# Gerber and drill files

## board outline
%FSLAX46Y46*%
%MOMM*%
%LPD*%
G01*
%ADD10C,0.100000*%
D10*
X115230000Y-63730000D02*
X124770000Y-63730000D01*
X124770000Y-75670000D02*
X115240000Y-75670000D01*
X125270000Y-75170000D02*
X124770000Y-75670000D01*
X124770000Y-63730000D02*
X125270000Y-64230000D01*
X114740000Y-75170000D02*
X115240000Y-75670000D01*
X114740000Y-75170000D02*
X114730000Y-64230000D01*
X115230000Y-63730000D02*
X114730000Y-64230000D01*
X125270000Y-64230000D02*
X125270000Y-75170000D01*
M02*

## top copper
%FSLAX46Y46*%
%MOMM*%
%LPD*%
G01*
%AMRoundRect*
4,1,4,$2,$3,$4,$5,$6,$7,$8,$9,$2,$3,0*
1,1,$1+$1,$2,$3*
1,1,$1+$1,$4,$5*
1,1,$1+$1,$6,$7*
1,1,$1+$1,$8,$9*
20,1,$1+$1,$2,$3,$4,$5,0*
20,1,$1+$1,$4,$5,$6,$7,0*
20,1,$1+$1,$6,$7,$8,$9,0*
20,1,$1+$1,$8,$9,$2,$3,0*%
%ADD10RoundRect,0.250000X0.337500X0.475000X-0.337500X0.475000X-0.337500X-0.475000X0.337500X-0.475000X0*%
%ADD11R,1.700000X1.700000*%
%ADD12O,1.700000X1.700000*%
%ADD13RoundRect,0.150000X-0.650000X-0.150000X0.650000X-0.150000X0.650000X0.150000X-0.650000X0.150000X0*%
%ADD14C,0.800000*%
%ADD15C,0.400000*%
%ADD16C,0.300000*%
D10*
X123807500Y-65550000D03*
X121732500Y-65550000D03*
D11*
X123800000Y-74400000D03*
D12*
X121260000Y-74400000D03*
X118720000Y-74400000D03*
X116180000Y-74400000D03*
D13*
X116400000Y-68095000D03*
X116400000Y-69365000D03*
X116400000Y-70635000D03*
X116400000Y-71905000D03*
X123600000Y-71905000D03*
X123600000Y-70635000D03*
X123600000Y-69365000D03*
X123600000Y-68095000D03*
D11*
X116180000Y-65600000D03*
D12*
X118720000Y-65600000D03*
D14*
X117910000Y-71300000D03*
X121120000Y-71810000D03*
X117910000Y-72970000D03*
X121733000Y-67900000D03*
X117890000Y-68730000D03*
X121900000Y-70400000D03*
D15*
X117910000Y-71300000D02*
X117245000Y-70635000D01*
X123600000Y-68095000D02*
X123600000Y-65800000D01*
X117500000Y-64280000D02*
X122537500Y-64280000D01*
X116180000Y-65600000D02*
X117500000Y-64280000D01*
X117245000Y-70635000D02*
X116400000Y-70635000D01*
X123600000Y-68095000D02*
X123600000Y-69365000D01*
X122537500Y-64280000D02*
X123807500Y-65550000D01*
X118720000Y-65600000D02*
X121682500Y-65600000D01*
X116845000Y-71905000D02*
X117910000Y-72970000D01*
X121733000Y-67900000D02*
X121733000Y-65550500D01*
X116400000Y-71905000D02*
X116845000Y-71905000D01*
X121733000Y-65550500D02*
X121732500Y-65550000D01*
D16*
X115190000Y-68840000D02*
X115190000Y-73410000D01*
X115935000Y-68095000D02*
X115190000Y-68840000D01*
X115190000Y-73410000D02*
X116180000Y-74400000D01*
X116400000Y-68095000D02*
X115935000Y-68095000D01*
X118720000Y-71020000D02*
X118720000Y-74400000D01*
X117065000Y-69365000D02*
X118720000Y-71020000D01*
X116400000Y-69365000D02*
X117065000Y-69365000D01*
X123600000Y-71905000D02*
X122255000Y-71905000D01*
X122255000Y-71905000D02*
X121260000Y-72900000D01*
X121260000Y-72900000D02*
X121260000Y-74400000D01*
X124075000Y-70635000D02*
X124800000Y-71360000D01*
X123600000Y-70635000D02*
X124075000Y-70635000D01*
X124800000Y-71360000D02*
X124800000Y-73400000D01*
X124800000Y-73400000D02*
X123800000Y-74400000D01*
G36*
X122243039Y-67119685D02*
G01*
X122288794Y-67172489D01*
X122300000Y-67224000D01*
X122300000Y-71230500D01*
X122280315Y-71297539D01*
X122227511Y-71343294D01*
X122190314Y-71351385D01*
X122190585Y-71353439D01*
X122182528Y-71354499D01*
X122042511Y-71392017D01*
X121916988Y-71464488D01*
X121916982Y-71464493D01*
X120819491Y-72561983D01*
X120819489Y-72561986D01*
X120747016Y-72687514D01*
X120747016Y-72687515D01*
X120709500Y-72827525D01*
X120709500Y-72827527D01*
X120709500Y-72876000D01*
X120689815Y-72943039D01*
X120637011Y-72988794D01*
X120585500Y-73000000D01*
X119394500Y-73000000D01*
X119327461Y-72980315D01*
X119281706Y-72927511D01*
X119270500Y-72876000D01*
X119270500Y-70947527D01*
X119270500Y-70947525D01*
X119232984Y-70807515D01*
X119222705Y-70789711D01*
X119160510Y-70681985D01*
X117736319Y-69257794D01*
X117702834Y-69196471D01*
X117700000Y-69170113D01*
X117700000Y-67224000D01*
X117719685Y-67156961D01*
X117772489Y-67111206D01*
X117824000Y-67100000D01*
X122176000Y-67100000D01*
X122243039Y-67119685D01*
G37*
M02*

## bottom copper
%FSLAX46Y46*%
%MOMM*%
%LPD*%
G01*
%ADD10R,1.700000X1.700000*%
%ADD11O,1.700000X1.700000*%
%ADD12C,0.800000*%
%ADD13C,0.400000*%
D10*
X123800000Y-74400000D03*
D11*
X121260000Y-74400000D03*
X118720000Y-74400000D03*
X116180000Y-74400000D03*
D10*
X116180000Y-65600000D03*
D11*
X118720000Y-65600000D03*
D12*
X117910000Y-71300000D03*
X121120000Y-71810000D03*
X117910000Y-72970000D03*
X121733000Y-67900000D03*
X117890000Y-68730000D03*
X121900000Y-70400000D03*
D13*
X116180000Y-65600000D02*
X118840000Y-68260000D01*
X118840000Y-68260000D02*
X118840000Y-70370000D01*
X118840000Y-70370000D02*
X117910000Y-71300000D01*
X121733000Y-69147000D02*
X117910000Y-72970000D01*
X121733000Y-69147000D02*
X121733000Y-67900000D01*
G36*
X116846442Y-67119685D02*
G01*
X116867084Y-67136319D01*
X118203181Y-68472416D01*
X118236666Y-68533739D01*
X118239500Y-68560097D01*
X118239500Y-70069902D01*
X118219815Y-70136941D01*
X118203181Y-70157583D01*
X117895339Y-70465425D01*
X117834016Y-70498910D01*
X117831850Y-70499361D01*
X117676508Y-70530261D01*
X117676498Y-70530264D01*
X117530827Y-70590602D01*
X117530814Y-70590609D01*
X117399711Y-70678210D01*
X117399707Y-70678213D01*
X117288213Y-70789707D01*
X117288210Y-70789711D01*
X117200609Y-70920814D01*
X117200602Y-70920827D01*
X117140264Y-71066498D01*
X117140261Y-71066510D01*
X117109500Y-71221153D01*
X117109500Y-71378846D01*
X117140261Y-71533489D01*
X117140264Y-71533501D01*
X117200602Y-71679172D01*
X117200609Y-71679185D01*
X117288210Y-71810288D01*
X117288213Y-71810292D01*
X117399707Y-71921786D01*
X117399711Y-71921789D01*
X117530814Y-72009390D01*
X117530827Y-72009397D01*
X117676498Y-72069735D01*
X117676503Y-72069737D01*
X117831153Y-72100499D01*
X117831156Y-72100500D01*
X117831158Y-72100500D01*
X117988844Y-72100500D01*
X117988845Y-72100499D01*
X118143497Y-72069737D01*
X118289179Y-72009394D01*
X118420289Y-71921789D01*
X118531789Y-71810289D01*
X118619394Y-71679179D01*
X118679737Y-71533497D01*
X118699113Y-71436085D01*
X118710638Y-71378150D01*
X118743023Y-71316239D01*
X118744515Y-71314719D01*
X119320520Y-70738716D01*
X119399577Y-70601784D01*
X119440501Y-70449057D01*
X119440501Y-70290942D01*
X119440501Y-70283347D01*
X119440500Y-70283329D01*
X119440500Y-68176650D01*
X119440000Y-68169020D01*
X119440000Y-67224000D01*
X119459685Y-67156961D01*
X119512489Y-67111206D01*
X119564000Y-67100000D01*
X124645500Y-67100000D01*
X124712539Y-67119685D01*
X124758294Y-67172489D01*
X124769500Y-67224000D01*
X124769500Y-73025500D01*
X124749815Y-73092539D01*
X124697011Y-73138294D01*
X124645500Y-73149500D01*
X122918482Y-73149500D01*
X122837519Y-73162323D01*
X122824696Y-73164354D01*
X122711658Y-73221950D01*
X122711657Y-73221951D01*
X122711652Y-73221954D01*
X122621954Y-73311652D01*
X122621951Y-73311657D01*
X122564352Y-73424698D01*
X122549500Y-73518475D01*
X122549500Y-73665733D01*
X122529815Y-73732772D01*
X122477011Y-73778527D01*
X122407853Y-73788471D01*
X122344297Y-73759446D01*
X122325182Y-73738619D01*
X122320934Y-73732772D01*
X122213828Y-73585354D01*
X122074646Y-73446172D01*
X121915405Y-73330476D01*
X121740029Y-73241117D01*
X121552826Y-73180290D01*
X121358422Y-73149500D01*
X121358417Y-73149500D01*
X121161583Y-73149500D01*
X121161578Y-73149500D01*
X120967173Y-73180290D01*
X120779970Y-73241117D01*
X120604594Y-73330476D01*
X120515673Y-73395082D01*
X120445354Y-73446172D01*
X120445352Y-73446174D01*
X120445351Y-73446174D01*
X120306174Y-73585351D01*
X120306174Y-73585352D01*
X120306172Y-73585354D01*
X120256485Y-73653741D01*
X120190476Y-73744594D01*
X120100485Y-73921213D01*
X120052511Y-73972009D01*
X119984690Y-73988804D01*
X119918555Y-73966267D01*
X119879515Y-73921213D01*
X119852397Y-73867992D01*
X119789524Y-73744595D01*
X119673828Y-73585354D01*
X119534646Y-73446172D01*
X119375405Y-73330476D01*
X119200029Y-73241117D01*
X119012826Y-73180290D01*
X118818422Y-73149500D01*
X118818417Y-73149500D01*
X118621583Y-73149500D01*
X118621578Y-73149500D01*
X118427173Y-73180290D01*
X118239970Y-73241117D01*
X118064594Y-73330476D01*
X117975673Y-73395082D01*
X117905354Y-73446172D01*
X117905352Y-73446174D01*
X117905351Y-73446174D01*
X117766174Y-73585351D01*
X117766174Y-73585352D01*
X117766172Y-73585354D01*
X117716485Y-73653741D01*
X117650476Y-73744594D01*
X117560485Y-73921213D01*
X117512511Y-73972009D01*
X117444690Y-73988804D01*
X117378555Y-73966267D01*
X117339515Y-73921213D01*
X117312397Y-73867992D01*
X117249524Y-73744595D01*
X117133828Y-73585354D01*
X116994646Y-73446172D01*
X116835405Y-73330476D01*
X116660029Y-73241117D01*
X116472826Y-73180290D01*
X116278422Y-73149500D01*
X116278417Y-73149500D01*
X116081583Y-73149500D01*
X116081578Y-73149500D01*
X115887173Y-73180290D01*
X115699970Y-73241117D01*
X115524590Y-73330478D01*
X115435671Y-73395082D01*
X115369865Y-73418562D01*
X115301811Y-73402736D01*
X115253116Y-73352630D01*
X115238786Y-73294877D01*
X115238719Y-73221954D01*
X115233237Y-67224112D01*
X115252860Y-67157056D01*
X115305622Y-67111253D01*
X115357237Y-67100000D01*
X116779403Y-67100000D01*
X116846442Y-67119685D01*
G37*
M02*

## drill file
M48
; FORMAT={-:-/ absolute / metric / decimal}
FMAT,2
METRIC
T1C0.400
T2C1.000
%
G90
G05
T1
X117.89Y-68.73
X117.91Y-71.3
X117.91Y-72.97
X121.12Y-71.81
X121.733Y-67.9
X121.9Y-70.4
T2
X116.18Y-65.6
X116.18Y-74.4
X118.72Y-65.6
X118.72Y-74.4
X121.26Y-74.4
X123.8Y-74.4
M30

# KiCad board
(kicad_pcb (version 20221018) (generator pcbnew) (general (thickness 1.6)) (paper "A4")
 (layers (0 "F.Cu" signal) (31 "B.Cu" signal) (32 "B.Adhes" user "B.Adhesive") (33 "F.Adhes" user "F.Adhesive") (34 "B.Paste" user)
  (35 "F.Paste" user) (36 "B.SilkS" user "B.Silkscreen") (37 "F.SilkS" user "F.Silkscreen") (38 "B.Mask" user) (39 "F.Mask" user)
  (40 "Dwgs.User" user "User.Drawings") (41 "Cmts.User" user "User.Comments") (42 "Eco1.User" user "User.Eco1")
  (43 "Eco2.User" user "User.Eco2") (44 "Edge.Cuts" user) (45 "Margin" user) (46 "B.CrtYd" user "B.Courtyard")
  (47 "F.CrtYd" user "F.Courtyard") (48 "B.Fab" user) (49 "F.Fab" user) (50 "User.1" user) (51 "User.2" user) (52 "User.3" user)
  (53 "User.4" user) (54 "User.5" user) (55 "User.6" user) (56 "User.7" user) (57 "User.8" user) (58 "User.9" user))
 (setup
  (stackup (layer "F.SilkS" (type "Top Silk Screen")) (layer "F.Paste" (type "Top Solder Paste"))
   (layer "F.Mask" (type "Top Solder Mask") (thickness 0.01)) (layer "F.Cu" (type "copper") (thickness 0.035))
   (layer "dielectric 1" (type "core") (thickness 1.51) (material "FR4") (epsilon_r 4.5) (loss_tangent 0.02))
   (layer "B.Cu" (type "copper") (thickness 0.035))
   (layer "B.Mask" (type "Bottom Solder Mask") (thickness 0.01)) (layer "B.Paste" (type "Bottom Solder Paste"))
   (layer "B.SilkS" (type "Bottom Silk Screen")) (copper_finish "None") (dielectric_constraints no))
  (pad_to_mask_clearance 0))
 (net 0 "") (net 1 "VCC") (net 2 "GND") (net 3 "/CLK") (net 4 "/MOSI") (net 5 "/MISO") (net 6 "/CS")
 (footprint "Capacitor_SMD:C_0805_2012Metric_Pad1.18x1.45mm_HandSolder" (layer "F.Cu") (at 122.77 65.55 180)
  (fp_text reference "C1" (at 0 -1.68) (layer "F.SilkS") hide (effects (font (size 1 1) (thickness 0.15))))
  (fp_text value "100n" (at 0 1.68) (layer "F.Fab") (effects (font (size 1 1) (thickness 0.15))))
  (pad "1" smd roundrect (at -1.0375 0 180) (size 1.175 1.45) (layers "F.Cu" "F.Paste" "F.Mask") (roundrect_rratio 0.2127659574)
   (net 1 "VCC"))
  (pad "2" smd roundrect (at 1.0375 0 180) (size 1.175 1.45) (layers "F.Cu" "F.Paste" "F.Mask") (roundrect_rratio 0.2127659574)
   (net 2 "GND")))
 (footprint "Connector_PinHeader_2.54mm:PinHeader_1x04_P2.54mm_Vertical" (layer "F.Cu") (at 123.8 74.4 -90)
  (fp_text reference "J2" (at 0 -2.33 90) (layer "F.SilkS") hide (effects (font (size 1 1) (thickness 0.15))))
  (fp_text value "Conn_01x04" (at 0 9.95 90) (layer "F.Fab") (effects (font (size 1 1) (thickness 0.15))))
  (pad "1" thru_hole rect (at 0 0 270) (size 1.7 1.7) (drill 1) (layers "*.Cu" "*.Mask") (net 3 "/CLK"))
  (pad "2" thru_hole oval (at 0 2.54 270) (size 1.7 1.7) (drill 1) (layers "*.Cu" "*.Mask") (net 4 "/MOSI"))
  (pad "3" thru_hole oval (at 0 5.08 270) (size 1.7 1.7) (drill 1) (layers "*.Cu" "*.Mask") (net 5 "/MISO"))
  (pad "4" thru_hole oval (at 0 7.62 270) (size 1.7 1.7) (drill 1) (layers "*.Cu" "*.Mask") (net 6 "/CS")))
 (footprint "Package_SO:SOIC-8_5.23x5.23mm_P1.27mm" (layer "F.Cu") (at 120 70)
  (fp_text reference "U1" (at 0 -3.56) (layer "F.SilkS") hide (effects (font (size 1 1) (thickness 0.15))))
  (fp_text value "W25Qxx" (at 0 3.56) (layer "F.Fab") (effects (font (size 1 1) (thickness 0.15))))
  (pad "1" smd roundrect (at -3.6 -1.905) (size 1.6 0.6) (layers "F.Cu" "F.Paste" "F.Mask") (roundrect_rratio 0.25) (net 6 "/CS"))
  (pad "2" smd roundrect (at -3.6 -0.635) (size 1.6 0.6) (layers "F.Cu" "F.Paste" "F.Mask") (roundrect_rratio 0.25) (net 5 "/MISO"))
  (pad "3" smd roundrect (at -3.6 0.635) (size 1.6 0.6) (layers "F.Cu" "F.Paste" "F.Mask") (roundrect_rratio 0.25) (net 1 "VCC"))
  (pad "4" smd roundrect (at -3.6 1.905) (size 1.6 0.6) (layers "F.Cu" "F.Paste" "F.Mask") (roundrect_rratio 0.25) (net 2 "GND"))
  (pad "5" smd roundrect (at 3.6 1.905) (size 1.6 0.6) (layers "F.Cu" "F.Paste" "F.Mask") (roundrect_rratio 0.25) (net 4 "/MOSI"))
  (pad "6" smd roundrect (at 3.6 0.635) (size 1.6 0.6) (layers "F.Cu" "F.Paste" "F.Mask") (roundrect_rratio 0.25) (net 3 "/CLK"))
  (pad "7" smd roundrect (at 3.6 -0.635) (size 1.6 0.6) (layers "F.Cu" "F.Paste" "F.Mask") (roundrect_rratio 0.25) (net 1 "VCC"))
  (pad "8" smd roundrect (at 3.6 -1.905) (size 1.6 0.6) (layers "F.Cu" "F.Paste" "F.Mask") (roundrect_rratio 0.25) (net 1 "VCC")))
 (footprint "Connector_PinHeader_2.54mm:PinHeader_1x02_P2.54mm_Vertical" (layer "F.Cu") (at 116.18 65.6 90)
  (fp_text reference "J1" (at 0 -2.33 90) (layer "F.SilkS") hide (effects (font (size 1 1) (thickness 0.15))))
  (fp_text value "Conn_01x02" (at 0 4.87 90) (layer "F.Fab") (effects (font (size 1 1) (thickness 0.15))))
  (pad "1" thru_hole rect (at 0 0 90) (size 1.7 1.7) (drill 1) (layers "*.Cu" "*.Mask") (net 1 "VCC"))
  (pad "2" thru_hole oval (at 0 2.54 90) (size 1.7 1.7) (drill 1) (layers "*.Cu" "*.Mask") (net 2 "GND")))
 (gr_line (start 115.23 63.73) (end 124.77 63.73) (stroke (width 0.1) (type default)) (layer "Edge.Cuts"))
 (gr_line (start 124.77 75.67) (end 115.24 75.67) (stroke (width 0.1) (type default)) (layer "Edge.Cuts"))
 (gr_line (start 125.27 75.17) (end 124.77 75.67) (stroke (width 0.1) (type default)) (layer "Edge.Cuts"))
 (gr_line (start 124.77 63.73) (end 125.27 64.23) (stroke (width 0.1) (type default)) (layer "Edge.Cuts"))
 (gr_line (start 114.74 75.17) (end 115.24 75.67) (stroke (width 0.1) (type default)) (layer "Edge.Cuts"))
 (gr_line (start 114.74 75.17) (end 114.73 64.23) (stroke (width 0.1) (type default)) (layer "Edge.Cuts"))
 (gr_line (start 115.23 63.73) (end 114.73 64.23) (stroke (width 0.1) (type default)) (layer "Edge.Cuts"))
 (gr_line (start 125.27 64.23) (end 125.27 75.17) (stroke (width 0.1) (type default)) (layer "Edge.Cuts"))
 (segment (start 117.91 71.3) (end 117.245 70.635) (width 0.4) (layer "F.Cu") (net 1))
 (segment (start 123.6 68.095) (end 123.6 65.8) (width 0.4) (layer "F.Cu") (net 1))
 (segment (start 117.5 64.28) (end 122.5375 64.28) (width 0.4) (layer "F.Cu") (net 1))
 (segment (start 116.18 65.6) (end 117.5 64.28) (width 0.4) (layer "F.Cu") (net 1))
 (segment (start 117.245 70.635) (end 116.4 70.635) (width 0.4) (layer "F.Cu") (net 1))
 (segment (start 123.6 68.095) (end 123.6 69.365) (width 0.4) (layer "F.Cu") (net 1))
 (segment (start 122.5375 64.28) (end 123.8075 65.55) (width 0.4) (layer "F.Cu") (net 1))
 (via (at 117.91 71.3) (size 0.8) (drill 0.4) (layers "F.Cu" "B.Cu") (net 1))
 (segment (start 116.18 65.6) (end 118.84 68.26) (width 0.4) (layer "B.Cu") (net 1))
 (segment (start 118.84 68.26) (end 118.84 70.37) (width 0.4) (layer "B.Cu") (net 1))
 (segment (start 118.84 70.37) (end 117.91 71.3) (width 0.4) (layer "B.Cu") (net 1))
 (segment (start 118.72 65.6) (end 121.6825 65.6) (width 0.4) (layer "F.Cu") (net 2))
 (segment (start 116.845 71.905) (end 117.91 72.97) (width 0.4) (layer "F.Cu") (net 2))
 (segment (start 121.733 67.9) (end 121.733 65.5505) (width 0.4) (layer "F.Cu") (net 2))
 (segment (start 116.4 71.905) (end 116.845 71.905) (width 0.4) (layer "F.Cu") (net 2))
 (segment (start 121.733 65.5505) (end 121.7325 65.55) (width 0.4) (layer "F.Cu") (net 2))
 (via (at 121.12 71.81) (size 0.8) (drill 0.4) (layers "F.Cu" "B.Cu") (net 2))
 (via (at 117.91 72.97) (size 0.8) (drill 0.4) (layers "F.Cu" "B.Cu") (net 2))
 (via (at 121.733 67.9) (size 0.8) (drill 0.4) (layers "F.Cu" "B.Cu") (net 2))
 (via (at 117.89 68.73) (size 0.8) (drill 0.4) (layers "F.Cu" "B.Cu") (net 2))
 (via (at 121.9 70.4) (size 0.8) (drill 0.4) (layers "F.Cu" "B.Cu") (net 2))
 (segment (start 121.733 69.147) (end 117.91 72.97) (width 0.4) (layer "B.Cu") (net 2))
 (segment (start 121.733 69.147) (end 121.733 67.9) (width 0.4) (layer "B.Cu") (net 2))
 (segment (start 115.19 68.84) (end 115.19 73.41) (width 0.3) (layer "F.Cu") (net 6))
 (segment (start 115.935 68.095) (end 115.19 68.84) (width 0.3) (layer "F.Cu") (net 6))
 (segment (start 115.19 73.41) (end 116.18 74.4) (width 0.3) (layer "F.Cu") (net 6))
 (segment (start 116.4 68.095) (end 115.935 68.095) (width 0.3) (layer "F.Cu") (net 6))
 (segment (start 118.72 71.02) (end 118.72 74.4) (width 0.3) (layer "F.Cu") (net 5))
 (segment (start 117.065 69.365) (end 118.72 71.02) (width 0.3) (layer "F.Cu") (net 5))
 (segment (start 116.4 69.365) (end 117.065 69.365) (width 0.3) (layer "F.Cu") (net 5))
 (segment (start 123.6 71.905) (end 122.255 71.905) (width 0.3) (layer "F.Cu") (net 4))
 (segment (start 122.255 71.905) (end 121.26 72.9) (width 0.3) (layer "F.Cu") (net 4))
 (segment (start 121.26 72.9) (end 121.26 74.4) (width 0.3) (layer "F.Cu") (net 4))
 (segment (start 124.075 70.635) (end 124.8 71.36) (width 0.3) (layer "F.Cu") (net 3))
 (segment (start 123.6 70.635) (end 124.075 70.635) (width 0.3) (layer "F.Cu") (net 3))
 (segment (start 124.8 71.36) (end 124.8 73.4) (width 0.3) (layer "F.Cu") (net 3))
 (segment (start 124.8 73.4) (end 123.8 74.4) (width 0.3) (layer "F.Cu") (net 3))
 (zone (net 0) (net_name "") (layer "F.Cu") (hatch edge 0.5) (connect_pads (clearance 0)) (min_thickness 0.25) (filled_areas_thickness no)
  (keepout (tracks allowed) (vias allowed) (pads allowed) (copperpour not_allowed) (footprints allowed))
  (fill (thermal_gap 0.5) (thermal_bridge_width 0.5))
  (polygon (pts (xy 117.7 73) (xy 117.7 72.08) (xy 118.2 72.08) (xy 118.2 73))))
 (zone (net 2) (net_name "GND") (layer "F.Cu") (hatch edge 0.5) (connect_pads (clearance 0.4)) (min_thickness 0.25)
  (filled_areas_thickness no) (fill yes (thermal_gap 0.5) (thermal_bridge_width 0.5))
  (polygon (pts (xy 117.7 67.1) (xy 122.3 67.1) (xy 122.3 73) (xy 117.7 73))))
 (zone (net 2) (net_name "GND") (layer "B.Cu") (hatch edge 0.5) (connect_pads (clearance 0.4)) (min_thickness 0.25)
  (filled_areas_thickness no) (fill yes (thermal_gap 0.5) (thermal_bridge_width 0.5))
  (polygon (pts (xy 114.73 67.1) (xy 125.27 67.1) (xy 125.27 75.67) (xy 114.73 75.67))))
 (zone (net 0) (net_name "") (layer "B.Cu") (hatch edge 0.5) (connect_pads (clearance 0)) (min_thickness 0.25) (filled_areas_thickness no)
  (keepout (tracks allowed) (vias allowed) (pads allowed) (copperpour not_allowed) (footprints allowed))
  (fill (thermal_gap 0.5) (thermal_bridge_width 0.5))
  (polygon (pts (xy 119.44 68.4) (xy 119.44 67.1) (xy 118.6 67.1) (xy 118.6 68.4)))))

